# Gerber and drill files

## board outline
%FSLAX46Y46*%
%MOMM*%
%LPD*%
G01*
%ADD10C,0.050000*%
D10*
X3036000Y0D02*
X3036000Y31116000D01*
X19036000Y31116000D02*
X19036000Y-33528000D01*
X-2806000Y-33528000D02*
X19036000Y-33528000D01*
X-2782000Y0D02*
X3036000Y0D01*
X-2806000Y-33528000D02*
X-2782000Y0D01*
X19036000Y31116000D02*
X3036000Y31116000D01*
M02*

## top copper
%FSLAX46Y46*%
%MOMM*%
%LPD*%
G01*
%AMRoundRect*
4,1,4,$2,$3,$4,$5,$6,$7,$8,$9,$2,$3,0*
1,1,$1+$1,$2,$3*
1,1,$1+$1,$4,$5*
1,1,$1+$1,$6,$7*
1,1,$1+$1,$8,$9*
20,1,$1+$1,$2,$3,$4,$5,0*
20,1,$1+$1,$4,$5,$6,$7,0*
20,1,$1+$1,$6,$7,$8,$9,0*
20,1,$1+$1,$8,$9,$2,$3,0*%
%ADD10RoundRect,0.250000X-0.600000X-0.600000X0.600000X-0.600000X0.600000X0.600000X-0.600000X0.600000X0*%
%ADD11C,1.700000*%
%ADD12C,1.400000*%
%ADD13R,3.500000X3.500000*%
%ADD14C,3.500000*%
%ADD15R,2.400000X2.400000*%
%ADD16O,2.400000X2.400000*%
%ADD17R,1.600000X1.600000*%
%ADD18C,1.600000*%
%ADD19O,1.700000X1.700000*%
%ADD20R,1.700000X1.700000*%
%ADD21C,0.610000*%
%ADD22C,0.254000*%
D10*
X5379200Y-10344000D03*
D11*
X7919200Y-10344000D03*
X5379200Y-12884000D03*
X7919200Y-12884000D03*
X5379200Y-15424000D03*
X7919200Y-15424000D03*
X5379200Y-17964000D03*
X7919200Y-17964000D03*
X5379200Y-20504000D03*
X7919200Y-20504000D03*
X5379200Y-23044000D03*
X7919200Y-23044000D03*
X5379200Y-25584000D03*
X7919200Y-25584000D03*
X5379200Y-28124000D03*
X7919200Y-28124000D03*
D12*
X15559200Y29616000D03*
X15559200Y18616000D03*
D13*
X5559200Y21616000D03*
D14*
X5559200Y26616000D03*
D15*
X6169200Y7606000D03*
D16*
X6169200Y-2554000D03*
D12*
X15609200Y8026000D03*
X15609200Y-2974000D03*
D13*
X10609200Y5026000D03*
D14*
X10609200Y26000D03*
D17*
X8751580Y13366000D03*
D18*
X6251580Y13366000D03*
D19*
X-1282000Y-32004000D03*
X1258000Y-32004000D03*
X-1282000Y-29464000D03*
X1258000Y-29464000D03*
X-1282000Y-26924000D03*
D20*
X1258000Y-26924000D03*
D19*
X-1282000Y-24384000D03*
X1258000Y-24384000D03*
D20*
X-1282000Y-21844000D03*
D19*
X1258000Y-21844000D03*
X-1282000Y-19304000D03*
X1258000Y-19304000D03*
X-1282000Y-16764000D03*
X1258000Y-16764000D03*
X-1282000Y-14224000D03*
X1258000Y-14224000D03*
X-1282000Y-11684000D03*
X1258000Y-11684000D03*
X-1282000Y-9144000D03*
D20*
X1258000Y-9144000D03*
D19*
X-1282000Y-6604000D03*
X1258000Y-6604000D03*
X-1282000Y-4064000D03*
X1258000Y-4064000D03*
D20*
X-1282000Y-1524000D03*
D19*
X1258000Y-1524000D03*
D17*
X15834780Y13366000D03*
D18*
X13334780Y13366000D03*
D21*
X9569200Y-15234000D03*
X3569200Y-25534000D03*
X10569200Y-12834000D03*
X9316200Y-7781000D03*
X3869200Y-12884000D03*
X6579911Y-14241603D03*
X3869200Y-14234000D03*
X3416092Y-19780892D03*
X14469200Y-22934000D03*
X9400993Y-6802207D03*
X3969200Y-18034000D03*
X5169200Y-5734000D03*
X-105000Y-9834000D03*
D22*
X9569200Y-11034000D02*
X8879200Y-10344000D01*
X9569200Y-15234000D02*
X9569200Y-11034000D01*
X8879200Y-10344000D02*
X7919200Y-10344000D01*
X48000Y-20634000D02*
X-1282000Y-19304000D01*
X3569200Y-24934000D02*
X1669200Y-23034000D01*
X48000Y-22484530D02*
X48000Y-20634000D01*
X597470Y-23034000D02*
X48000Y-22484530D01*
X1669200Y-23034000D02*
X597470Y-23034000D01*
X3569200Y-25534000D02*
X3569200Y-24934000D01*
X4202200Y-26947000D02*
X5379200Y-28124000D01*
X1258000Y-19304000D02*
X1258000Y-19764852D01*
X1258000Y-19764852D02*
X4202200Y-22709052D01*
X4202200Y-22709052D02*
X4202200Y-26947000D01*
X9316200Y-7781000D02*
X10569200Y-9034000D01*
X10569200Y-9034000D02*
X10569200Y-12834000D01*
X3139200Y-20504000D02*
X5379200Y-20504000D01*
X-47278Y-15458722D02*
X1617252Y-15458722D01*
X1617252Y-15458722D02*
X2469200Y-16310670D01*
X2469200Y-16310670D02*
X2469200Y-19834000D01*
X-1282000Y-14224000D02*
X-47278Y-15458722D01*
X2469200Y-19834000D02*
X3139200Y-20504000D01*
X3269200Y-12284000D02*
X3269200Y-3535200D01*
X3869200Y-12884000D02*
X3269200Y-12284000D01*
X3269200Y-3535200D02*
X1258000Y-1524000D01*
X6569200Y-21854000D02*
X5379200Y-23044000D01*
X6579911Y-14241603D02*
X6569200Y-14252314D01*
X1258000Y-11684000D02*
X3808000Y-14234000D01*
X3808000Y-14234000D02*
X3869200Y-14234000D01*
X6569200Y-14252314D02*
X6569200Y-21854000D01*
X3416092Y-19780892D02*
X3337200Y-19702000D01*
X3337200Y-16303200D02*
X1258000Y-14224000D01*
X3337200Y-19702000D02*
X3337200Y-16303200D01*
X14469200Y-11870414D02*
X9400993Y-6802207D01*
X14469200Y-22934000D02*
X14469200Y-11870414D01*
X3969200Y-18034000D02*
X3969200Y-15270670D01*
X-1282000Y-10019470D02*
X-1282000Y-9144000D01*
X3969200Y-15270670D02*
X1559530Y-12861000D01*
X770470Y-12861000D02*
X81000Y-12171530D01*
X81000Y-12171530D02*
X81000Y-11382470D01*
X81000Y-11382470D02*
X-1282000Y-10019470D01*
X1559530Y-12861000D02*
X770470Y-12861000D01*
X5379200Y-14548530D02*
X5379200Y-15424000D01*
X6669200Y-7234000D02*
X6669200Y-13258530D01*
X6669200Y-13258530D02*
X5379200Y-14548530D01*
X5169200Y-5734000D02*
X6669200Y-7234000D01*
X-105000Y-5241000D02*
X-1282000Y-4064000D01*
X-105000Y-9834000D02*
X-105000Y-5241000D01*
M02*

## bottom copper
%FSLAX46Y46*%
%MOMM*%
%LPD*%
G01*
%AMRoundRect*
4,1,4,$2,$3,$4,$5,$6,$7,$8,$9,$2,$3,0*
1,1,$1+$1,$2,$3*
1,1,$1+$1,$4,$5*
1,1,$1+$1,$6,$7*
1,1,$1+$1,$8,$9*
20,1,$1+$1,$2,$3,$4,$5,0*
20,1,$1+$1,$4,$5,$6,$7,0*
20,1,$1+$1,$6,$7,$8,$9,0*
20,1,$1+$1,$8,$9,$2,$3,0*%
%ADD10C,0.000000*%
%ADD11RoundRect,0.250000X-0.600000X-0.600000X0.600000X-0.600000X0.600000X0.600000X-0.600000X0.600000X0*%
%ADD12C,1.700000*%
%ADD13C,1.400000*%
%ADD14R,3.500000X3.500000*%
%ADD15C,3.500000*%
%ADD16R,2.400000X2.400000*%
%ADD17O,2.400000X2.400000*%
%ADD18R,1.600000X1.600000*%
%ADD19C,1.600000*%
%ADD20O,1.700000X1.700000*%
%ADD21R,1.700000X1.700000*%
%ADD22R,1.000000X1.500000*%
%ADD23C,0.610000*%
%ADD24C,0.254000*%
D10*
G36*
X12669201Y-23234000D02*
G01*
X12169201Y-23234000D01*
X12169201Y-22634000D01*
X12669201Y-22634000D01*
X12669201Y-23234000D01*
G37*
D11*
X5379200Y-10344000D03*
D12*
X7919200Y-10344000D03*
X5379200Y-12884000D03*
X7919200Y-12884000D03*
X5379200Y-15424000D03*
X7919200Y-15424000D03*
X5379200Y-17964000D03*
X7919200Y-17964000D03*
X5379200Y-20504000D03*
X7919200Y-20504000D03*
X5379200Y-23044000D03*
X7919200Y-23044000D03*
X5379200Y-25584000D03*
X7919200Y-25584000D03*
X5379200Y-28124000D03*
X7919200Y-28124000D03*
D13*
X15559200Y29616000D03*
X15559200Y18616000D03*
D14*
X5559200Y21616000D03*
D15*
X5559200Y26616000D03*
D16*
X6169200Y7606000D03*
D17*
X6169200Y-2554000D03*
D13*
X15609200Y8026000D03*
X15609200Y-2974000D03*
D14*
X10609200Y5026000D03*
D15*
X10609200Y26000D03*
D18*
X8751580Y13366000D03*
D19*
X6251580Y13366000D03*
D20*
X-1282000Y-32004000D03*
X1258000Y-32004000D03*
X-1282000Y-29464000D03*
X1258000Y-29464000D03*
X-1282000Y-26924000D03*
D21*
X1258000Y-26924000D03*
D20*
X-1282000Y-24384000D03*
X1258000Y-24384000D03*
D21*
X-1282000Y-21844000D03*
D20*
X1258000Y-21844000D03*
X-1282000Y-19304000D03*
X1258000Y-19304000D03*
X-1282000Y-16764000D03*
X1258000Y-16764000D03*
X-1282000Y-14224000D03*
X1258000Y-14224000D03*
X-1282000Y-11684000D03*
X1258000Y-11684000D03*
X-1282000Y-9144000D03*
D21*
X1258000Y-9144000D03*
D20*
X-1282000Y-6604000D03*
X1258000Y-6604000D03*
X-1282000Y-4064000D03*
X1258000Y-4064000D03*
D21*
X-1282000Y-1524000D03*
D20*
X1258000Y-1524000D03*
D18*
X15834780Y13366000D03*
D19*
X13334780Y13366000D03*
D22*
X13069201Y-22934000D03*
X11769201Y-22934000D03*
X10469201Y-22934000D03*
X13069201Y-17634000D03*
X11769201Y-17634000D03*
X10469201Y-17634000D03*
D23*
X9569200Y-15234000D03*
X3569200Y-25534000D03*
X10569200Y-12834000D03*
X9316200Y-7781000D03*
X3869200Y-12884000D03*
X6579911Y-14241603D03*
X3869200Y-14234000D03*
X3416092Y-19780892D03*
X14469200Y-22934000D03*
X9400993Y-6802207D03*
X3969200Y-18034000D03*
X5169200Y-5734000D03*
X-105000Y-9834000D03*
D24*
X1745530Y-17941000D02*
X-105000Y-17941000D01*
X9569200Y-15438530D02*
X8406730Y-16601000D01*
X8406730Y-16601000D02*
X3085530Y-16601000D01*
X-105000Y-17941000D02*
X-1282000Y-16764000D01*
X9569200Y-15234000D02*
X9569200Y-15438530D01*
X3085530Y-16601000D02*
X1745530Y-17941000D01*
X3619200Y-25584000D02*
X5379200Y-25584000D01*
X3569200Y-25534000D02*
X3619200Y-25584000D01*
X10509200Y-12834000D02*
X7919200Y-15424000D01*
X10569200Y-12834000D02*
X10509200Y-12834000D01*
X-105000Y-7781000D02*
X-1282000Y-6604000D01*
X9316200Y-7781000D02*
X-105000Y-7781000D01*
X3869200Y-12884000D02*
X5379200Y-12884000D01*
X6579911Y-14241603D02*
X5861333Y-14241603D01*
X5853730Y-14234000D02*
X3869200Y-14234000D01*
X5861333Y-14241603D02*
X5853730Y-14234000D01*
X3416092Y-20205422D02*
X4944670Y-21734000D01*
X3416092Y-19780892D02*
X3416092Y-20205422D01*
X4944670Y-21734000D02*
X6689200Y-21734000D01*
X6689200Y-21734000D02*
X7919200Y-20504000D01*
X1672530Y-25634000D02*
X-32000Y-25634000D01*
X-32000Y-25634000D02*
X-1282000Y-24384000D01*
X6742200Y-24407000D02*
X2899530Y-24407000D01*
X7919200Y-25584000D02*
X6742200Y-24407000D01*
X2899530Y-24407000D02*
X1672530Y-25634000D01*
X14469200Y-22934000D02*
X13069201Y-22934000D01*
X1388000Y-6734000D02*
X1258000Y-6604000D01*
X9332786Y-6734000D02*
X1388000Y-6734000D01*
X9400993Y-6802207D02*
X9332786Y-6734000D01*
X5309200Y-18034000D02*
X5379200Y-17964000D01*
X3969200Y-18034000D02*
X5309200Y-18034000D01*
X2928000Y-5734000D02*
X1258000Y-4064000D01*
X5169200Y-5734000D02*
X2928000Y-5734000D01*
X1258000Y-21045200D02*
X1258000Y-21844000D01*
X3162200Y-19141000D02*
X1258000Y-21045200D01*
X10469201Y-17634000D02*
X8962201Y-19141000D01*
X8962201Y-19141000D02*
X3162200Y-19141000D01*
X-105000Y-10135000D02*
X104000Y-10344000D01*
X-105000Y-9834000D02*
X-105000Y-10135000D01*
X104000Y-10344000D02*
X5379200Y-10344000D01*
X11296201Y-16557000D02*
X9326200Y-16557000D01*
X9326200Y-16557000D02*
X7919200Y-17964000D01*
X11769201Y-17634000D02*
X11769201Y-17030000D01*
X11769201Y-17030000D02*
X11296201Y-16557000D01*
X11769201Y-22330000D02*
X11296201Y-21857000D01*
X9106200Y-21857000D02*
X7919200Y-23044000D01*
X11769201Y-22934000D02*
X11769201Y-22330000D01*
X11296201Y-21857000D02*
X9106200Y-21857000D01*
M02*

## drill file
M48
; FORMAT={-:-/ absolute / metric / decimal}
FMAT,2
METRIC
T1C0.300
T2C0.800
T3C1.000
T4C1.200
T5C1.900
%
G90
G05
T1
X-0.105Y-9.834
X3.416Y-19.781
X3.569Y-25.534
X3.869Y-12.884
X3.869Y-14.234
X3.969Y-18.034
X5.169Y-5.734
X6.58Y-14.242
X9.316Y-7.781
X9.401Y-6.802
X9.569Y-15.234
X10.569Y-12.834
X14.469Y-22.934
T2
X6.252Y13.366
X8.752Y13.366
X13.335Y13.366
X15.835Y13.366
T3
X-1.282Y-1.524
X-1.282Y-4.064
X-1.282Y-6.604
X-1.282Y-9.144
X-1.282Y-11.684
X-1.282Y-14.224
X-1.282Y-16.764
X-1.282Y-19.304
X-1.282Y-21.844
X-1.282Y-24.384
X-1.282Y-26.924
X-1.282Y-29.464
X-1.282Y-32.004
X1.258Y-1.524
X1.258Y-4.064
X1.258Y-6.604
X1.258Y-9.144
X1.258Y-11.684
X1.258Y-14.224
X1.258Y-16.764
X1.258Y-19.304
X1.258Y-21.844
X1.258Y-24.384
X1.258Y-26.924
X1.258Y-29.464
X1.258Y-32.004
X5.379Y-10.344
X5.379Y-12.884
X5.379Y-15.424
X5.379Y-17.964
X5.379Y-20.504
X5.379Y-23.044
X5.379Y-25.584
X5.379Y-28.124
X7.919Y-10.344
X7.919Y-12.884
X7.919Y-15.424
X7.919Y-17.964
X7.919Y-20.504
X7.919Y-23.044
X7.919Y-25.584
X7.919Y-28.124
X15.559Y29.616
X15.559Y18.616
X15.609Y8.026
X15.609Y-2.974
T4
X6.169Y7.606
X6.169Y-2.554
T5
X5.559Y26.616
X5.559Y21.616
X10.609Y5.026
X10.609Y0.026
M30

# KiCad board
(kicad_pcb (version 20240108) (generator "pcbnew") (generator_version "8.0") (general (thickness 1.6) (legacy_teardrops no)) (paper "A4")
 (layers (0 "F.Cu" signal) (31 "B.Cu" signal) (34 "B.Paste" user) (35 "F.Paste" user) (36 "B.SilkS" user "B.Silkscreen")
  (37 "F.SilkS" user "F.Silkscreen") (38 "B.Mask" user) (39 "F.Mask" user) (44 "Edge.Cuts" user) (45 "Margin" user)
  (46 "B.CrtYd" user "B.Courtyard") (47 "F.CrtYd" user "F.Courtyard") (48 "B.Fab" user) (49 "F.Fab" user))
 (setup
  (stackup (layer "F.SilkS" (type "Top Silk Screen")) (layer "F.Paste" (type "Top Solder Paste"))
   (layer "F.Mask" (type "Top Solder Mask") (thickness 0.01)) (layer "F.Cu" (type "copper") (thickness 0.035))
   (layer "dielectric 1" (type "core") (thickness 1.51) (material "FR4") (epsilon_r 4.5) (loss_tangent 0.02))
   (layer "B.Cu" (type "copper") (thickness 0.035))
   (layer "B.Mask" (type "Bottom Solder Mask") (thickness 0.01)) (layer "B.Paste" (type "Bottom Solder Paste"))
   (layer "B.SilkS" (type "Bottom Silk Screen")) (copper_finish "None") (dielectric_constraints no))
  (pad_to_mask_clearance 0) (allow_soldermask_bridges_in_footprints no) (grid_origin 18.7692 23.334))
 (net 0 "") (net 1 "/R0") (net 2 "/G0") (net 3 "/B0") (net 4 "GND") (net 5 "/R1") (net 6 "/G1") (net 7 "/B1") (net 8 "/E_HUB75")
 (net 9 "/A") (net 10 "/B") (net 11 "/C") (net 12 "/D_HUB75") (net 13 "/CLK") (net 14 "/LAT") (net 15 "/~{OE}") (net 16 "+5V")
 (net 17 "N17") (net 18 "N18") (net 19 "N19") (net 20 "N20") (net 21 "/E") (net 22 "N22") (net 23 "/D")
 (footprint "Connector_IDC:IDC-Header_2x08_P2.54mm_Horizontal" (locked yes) (layer "F.Cu") (at 5.3792 10.344)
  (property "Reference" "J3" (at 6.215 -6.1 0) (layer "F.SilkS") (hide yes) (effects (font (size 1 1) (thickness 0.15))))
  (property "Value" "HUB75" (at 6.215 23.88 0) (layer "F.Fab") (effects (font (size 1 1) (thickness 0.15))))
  (pad "1" thru_hole roundrect (at 0 0) (size 1.7 1.7) (drill 1) (layers "*.Cu" "*.Mask") (remove_unused_layers no)
   (roundrect_rratio 0.147059) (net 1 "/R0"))
  (pad "2" thru_hole circle (at 2.54 0) (size 1.7 1.7) (drill 1) (layers "*.Cu" "*.Mask") (remove_unused_layers no) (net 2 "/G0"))
  (pad "3" thru_hole circle (at 0 2.54) (size 1.7 1.7) (drill 1) (layers "*.Cu" "*.Mask") (remove_unused_layers no) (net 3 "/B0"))
  (pad "4" thru_hole circle (at 2.54 2.54) (size 1.7 1.7) (drill 1) (layers "*.Cu" "*.Mask") (remove_unused_layers no) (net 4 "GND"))
  (pad "5" thru_hole circle (at 0 5.08) (size 1.7 1.7) (drill 1) (layers "*.Cu" "*.Mask") (remove_unused_layers no) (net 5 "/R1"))
  (pad "6" thru_hole circle (at 2.54 5.08) (size 1.7 1.7) (drill 1) (layers "*.Cu" "*.Mask") (remove_unused_layers no) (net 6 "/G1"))
  (pad "7" thru_hole circle (at 0 7.62) (size 1.7 1.7) (drill 1) (layers "*.Cu" "*.Mask") (remove_unused_layers no) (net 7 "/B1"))
  (pad "8" thru_hole circle (at 2.54 7.62) (size 1.7 1.7) (drill 1) (layers "*.Cu" "*.Mask") (remove_unused_layers no) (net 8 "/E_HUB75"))
  (pad "9" thru_hole circle (at 0 10.16) (size 1.7 1.7) (drill 1) (layers "*.Cu" "*.Mask") (remove_unused_layers no) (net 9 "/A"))
  (pad "10" thru_hole circle (at 2.54 10.16) (size 1.7 1.7) (drill 1) (layers "*.Cu" "*.Mask") (remove_unused_layers no) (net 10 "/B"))
  (pad "11" thru_hole circle (at 0 12.7) (size 1.7 1.7) (drill 1) (layers "*.Cu" "*.Mask") (remove_unused_layers no) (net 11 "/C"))
  (pad "12" thru_hole circle (at 2.54 12.7) (size 1.7 1.7) (drill 1) (layers "*.Cu" "*.Mask") (remove_unused_layers no) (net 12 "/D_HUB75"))
  (pad "13" thru_hole circle (at 0 15.24) (size 1.7 1.7) (drill 1) (layers "*.Cu" "*.Mask") (remove_unused_layers no) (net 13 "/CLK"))
  (pad "14" thru_hole circle (at 2.54 15.24) (size 1.7 1.7) (drill 1) (layers "*.Cu" "*.Mask") (remove_unused_layers no) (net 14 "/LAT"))
  (pad "15" thru_hole circle (at 0 17.78) (size 1.7 1.7) (drill 1) (layers "*.Cu" "*.Mask") (remove_unused_layers no) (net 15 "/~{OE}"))
  (pad "16" thru_hole circle (at 2.54 17.78) (size 1.7 1.7) (drill 1) (layers "*.Cu" "*.Mask") (remove_unused_layers no) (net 4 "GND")))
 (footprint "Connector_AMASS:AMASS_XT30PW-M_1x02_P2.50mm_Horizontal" (layer "F.Cu") (at 5.5592 -21.616 -90)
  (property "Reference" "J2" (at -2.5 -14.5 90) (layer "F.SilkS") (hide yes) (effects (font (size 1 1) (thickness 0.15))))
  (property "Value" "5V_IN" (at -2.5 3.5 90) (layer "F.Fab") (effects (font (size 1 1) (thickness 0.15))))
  (pad "" thru_hole circle (at -8 -10 270) (size 1.4 1.4) (drill 1) (layers "*.Cu" "*.Mask") (remove_unused_layers no))
  (pad "" thru_hole circle (at 3 -10 270) (size 1.4 1.4) (drill 1) (layers "*.Cu" "*.Mask") (remove_unused_layers no))
  (pad "1" thru_hole rect (at 0 0 270) (size 3.5 3.5) (drill 1.9) (layers "*.Cu" "*.Mask") (remove_unused_layers no) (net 4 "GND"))
  (pad "2" thru_hole circle (at -5 0 270) (size 3.5 3.5) (drill 1.9) (layers "*.Cu" "*.Mask") (remove_unused_layers no) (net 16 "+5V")))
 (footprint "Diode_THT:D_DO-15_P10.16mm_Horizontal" (layer "F.Cu") (at 6.1692 -7.606 -90)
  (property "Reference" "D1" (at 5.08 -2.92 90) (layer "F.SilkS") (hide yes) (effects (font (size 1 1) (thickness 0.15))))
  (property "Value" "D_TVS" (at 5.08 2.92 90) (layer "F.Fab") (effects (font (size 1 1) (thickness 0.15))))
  (pad "1" thru_hole rect (at 0 0 270) (size 2.4 2.4) (drill 1.2) (layers "*.Cu" "*.Mask") (remove_unused_layers no) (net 4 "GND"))
  (pad "2" thru_hole oval (at 10.16 0 270) (size 2.4 2.4) (drill 1.2) (layers "*.Cu" "*.Mask") (remove_unused_layers no) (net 16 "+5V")))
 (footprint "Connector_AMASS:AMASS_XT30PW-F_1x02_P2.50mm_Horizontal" (layer "F.Cu") (at 10.6092 -5.026 -90)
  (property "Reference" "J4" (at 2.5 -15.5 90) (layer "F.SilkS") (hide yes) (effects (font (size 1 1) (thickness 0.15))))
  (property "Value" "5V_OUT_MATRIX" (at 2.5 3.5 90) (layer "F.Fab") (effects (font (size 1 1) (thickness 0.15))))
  (pad "" thru_hole circle (at -3 -5) (size 1.4 1.4) (drill 1) (layers "*.Cu" "*.Mask") (remove_unused_layers no))
  (pad "" thru_hole circle (at 8 -5 270) (size 1.4 1.4) (drill 1) (layers "*.Cu" "*.Mask") (remove_unused_layers no))
  (pad "1" thru_hole rect (at 0 0 270) (size 3.5 3.5) (drill 1.9) (layers "*.Cu" "*.Mask") (remove_unused_layers no) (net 4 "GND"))
  (pad "2" thru_hole circle (at 5 0 270) (size 3.5 3.5) (drill 1.9) (layers "*.Cu" "*.Mask") (remove_unused_layers no) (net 16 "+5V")))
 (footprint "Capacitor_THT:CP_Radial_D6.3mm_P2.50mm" (layer "F.Cu") (at 8.75158 -13.366 180)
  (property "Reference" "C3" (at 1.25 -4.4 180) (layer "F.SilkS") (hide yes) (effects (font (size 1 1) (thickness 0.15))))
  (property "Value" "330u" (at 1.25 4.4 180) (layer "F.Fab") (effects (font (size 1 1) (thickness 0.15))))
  (pad "1" thru_hole rect (at 0 0 180) (size 1.6 1.6) (drill 0.8) (layers "*.Cu" "*.Mask") (remove_unused_layers no) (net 16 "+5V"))
  (pad "2" thru_hole circle (at 2.5 0 180) (size 1.6 1.6) (drill 0.8) (layers "*.Cu" "*.Mask") (remove_unused_layers no) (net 4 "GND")))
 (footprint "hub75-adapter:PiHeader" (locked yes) (layer "F.Cu") (at -1.282 1.524)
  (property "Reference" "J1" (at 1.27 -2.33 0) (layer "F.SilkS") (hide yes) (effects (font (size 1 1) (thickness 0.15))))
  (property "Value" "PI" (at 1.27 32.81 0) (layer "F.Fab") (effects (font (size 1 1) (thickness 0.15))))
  (pad "1" thru_hole oval (at 0 30.48 180) (size 1.7 1.7) (drill 1) (layers "*.Cu" "*.Mask") (remove_unused_layers no) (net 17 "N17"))
  (pad "2" thru_hole oval (at 2.54 30.48 180) (size 1.7 1.7) (drill 1) (layers "*.Cu" "*.Mask") (remove_unused_layers no) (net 16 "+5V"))
  (pad "3" thru_hole oval (at 0 27.94 180) (size 1.7 1.7) (drill 1) (layers "*.Cu" "*.Mask") (remove_unused_layers no) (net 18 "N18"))
  (pad "4" thru_hole oval (at 2.54 27.94 180) (size 1.7 1.7) (drill 1) (layers "*.Cu" "*.Mask") (remove_unused_layers no) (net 16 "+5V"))
  (pad "5" thru_hole oval (at 0 25.4 180) (size 1.7 1.7) (drill 1) (layers "*.Cu" "*.Mask") (remove_unused_layers no) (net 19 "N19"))
  (pad "6" thru_hole rect (at 2.54 25.4 180) (size 1.7 1.7) (drill 1) (layers "*.Cu" "*.Mask") (remove_unused_layers no) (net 4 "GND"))
  (pad "7" thru_hole oval (at 0 22.86 180) (size 1.7 1.7) (drill 1) (layers "*.Cu" "*.Mask") (remove_unused_layers no) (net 14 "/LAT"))
  (pad "8" thru_hole oval (at 2.54 22.86 180) (size 1.7 1.7) (drill 1) (layers "*.Cu" "*.Mask") (remove_unused_layers no) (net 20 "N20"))
  (pad "9" thru_hole rect (at 0 20.32 180) (size 1.7 1.7) (drill 1) (layers "*.Cu" "*.Mask") (remove_unused_layers no) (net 4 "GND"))
  (pad "10" thru_hole oval (at 2.54 20.32 180) (size 1.7 1.7) (drill 1) (layers "*.Cu" "*.Mask") (remove_unused_layers no) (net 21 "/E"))
  (pad "11" thru_hole oval (at 0 17.78 180) (size 1.7 1.7) (drill 1) (layers "*.Cu" "*.Mask") (remove_unused_layers no) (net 13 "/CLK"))
  (pad "12" thru_hole oval (at 2.54 17.78 180) (size 1.7 1.7) (drill 1) (layers "*.Cu" "*.Mask") (remove_unused_layers no) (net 15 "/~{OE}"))
  (pad "13" thru_hole oval (at 0 15.24 180) (size 1.7 1.7) (drill 1) (layers "*.Cu" "*.Mask") (remove_unused_layers no) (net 2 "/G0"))
  (pad "14" thru_hole oval (at 2.54 15.24 180) (size 1.7 1.7) (drill 1) (layers "*.Cu" "*.Mask") (remove_unused_layers no) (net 4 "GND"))
  (pad "15" thru_hole oval (at 0 12.7 180) (size 1.7 1.7) (drill 1) (layers "*.Cu" "*.Mask") (remove_unused_layers no) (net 9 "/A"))
  (pad "16" thru_hole oval (at 2.54 12.7 180) (size 1.7 1.7) (drill 1) (layers "*.Cu" "*.Mask") (remove_unused_layers no) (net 10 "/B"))
  (pad "17" thru_hole oval (at 0 10.16 180) (size 1.7 1.7) (drill 1) (layers "*.Cu" "*.Mask") (remove_unused_layers no) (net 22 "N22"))
  (pad "18" thru_hole oval (at 2.54 10.16 180) (size 1.7 1.7) (drill 1) (layers "*.Cu" "*.Mask") (remove_unused_layers no) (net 11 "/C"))
  (pad "19" thru_hole oval (at 0 7.62 180) (size 1.7 1.7) (drill 1) (layers "*.Cu" "*.Mask") (remove_unused_layers no) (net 7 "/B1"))
  (pad "20" thru_hole rect (at 2.54 7.62 180) (size 1.7 1.7) (drill 1) (layers "*.Cu" "*.Mask") (remove_unused_layers no) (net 4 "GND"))
  (pad "21" thru_hole oval (at 0 5.08 180) (size 1.7 1.7) (drill 1) (layers "*.Cu" "*.Mask") (remove_unused_layers no) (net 6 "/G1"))
  (pad "22" thru_hole oval (at 2.54 5.08 180) (size 1.7 1.7) (drill 1) (layers "*.Cu" "*.Mask") (remove_unused_layers no) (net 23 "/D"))
  (pad "23" thru_hole oval (at 0 2.54 180) (size 1.7 1.7) (drill 1) (layers "*.Cu" "*.Mask") (remove_unused_layers no) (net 1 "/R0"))
  (pad "24" thru_hole oval (at 2.54 2.54 180) (size 1.7 1.7) (drill 1) (layers "*.Cu" "*.Mask") (remove_unused_layers no) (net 5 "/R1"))
  (pad "25" thru_hole rect (at 0 0 180) (size 1.7 1.7) (drill 1) (layers "*.Cu" "*.Mask") (remove_unused_layers no) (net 4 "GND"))
  (pad "26" thru_hole oval (at 2.54 0 180) (size 1.7 1.7) (drill 1) (layers "*.Cu" "*.Mask") (remove_unused_layers no) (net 3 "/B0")))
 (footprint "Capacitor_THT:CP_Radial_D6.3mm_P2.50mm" (layer "F.Cu") (at 15.83478 -13.366 180)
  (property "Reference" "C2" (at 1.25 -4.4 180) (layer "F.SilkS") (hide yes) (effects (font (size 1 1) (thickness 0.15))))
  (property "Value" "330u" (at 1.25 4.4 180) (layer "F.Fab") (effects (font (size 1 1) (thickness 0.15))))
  (pad "1" thru_hole rect (at 0 0 180) (size 1.6 1.6) (drill 0.8) (layers "*.Cu" "*.Mask") (remove_unused_layers no) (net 16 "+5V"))
  (pad "2" thru_hole circle (at 2.5 0 180) (size 1.6 1.6) (drill 0.8) (layers "*.Cu" "*.Mask") (remove_unused_layers no) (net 4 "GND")))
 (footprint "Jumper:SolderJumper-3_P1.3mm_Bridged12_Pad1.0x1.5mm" (layer "B.Cu") (at 11.769201 22.934 180)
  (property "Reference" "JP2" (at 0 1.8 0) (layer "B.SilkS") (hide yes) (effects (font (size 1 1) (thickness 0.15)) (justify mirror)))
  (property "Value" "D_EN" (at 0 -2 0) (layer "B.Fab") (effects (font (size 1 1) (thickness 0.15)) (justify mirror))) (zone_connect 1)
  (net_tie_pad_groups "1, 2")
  (fp_poly (pts (xy -0.9 0.3) (xy -0.4 0.3) (xy -0.4 -0.3) (xy -0.9 -0.3)) (stroke (width 0) (type solid)) (fill solid) (layer "B.Cu"))
  (pad "1" smd rect (at -1.3 0 180) (size 1 1.5) (layers "B.Cu" "B.Mask") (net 23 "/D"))
  (pad "2" smd rect (at 0 0 180) (size 1 1.5) (layers "B.Cu" "B.Mask") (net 12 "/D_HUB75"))
  (pad "3" smd rect (at 1.3 0 180) (size 1 1.5) (layers "B.Cu" "B.Mask") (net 4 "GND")))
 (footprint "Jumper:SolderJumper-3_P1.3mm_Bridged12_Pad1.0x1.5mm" (layer "B.Cu") (at 11.769201 17.634 180)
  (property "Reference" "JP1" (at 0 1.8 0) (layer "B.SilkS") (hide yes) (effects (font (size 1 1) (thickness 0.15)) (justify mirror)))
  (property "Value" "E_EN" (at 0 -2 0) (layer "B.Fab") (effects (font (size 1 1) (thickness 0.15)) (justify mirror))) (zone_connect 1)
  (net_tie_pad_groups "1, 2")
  (pad "1" smd rect (at -1.3 0 180) (size 1 1.5) (layers "B.Cu" "B.Mask") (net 4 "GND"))
  (pad "2" smd rect (at 0 0 180) (size 1 1.5) (layers "B.Cu" "B.Mask") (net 8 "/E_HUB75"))
  (pad "3" smd rect (at 1.3 0 180) (size 1 1.5) (layers "B.Cu" "B.Mask") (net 21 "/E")))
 (gr_line (start 3.036 0) (end 3.036 -31.116) (stroke (width 0.05) (type default)) (layer "Edge.Cuts"))
 (gr_line (start 19.036 -31.116) (end 19.036 33.528) (stroke (width 0.05) (type default)) (layer "Edge.Cuts"))
 (gr_line (start -2.806 33.528) (end 19.036 33.528) (stroke (width 0.05) (type default)) (layer "Edge.Cuts"))
 (gr_line (start -2.782 0) (end 3.036 0) (stroke (width 0.05) (type default)) (layer "Edge.Cuts"))
 (gr_line (start -2.806 33.528) (end -2.782 0) (locked yes) (stroke (width 0.05) (type default)) (layer "Edge.Cuts"))
 (gr_line (start 19.036 -31.116) (end 3.036 -31.116) (stroke (width 0.05) (type default)) (layer "Edge.Cuts"))
 (segment (start 9.5692 11.034) (end 8.8792 10.344) (width 0.254) (layer "F.Cu") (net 2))
 (segment (start 9.5692 15.234) (end 9.5692 11.034) (width 0.254) (layer "F.Cu") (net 2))
 (segment (start 8.8792 10.344) (end 7.9192 10.344) (width 0.254) (layer "F.Cu") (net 2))
 (via (at 9.5692 15.234) (size 0.61) (drill 0.3) (layers "F.Cu" "B.Cu") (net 2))
 (segment (start 1.74553 17.941) (end -0.105 17.941) (width 0.254) (layer "B.Cu") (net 2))
 (segment (start 9.5692 15.43853) (end 8.40673 16.601) (width 0.254) (layer "B.Cu") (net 2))
 (segment (start 8.40673 16.601) (end 3.08553 16.601) (width 0.254) (layer "B.Cu") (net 2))
 (segment (start -0.105 17.941) (end -1.282 16.764) (width 0.254) (layer "B.Cu") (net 2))
 (segment (start 9.5692 15.234) (end 9.5692 15.43853) (width 0.254) (layer "B.Cu") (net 2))
 (segment (start 3.08553 16.601) (end 1.74553 17.941) (width 0.254) (layer "B.Cu") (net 2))
 (segment (start 0.048 20.634) (end -1.282 19.304) (width 0.254) (layer "F.Cu") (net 13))
 (segment (start 3.5692 24.934) (end 1.6692 23.034) (width 0.254) (layer "F.Cu") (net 13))
 (segment (start 0.048 22.48453) (end 0.048 20.634) (width 0.254) (layer "F.Cu") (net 13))
 (segment (start 0.59747 23.034) (end 0.048 22.48453) (width 0.254) (layer "F.Cu") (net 13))
 (segment (start 1.6692 23.034) (end 0.59747 23.034) (width 0.254) (layer "F.Cu") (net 13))
 (segment (start 3.5692 25.534) (end 3.5692 24.934) (width 0.254) (layer "F.Cu") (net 13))
 (via (at 3.5692 25.534) (size 0.61) (drill 0.3) (layers "F.Cu" "B.Cu") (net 13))
 (segment (start 3.6192 25.584) (end 5.3792 25.584) (width 0.254) (layer "B.Cu") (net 13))
 (segment (start 3.5692 25.534) (end 3.6192 25.584) (width 0.254) (layer "B.Cu") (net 13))
 (segment (start 4.2022 26.947) (end 5.3792 28.124) (width 0.254) (layer "F.Cu") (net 15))
 (segment (start 1.258 19.304) (end 1.258 19.764852) (width 0.254) (layer "F.Cu") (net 15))
 (segment (start 1.258 19.764852) (end 4.2022 22.709052) (width 0.254) (layer "F.Cu") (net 15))
 (segment (start 4.2022 22.709052) (end 4.2022 26.947) (width 0.254) (layer "F.Cu") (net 15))
 (segment (start 9.3162 7.781) (end 10.5692 9.034) (width 0.254) (layer "F.Cu") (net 6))
 (segment (start 10.5692 9.034) (end 10.5692 12.834) (width 0.254) (layer "F.Cu") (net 6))
 (via (at 10.5692 12.834) (size 0.61) (drill 0.3) (layers "F.Cu" "B.Cu") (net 6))
 (via (at 9.3162 7.781) (size 0.61) (drill 0.3) (layers "F.Cu" "B.Cu") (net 6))
 (segment (start 10.5092 12.834) (end 7.9192 15.424) (width 0.254) (layer "B.Cu") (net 6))
 (segment (start 10.5692 12.834) (end 10.5092 12.834) (width 0.254) (layer "B.Cu") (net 6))
 (segment (start -0.105 7.781) (end -1.282 6.604) (width 0.254) (layer "B.Cu") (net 6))
 (segment (start 9.3162 7.781) (end -0.105 7.781) (width 0.254) (layer "B.Cu") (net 6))
 (segment (start 3.1392 20.504) (end 5.3792 20.504) (width 0.254) (layer "F.Cu") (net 9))
 (segment (start -0.047278 15.458722) (end 1.617252 15.458722) (width 0.254) (layer "F.Cu") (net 9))
 (segment (start 1.617252 15.458722) (end 2.4692 16.31067) (width 0.254) (layer "F.Cu") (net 9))
 (segment (start 2.4692 16.31067) (end 2.4692 19.834) (width 0.254) (layer "F.Cu") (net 9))
 (segment (start -1.282 14.224) (end -0.047278 15.458722) (width 0.254) (layer "F.Cu") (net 9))
 (segment (start 2.4692 19.834) (end 3.1392 20.504) (width 0.254) (layer "F.Cu") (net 9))
 (segment (start 3.2692 12.284) (end 3.2692 3.5352) (width 0.254) (layer "F.Cu") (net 3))
 (segment (start 3.8692 12.884) (end 3.2692 12.284) (width 0.254) (layer "F.Cu") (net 3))
 (segment (start 3.2692 3.5352) (end 1.258 1.524) (width 0.254) (layer "F.Cu") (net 3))
 (via (at 3.8692 12.884) (size 0.61) (drill 0.3) (layers "F.Cu" "B.Cu") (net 3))
 (segment (start 3.8692 12.884) (end 5.3792 12.884) (width 0.254) (layer "B.Cu") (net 3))
 (segment (start 6.5692 21.854) (end 5.3792 23.044) (width 0.254) (layer "F.Cu") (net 11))
 (segment (start 6.579911 14.241603) (end 6.5692 14.252314) (width 0.254) (layer "F.Cu") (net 11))
 (segment (start 1.258 11.684) (end 3.808 14.234) (width 0.254) (layer "F.Cu") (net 11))
 (segment (start 3.808 14.234) (end 3.8692 14.234) (width 0.254) (layer "F.Cu") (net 11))
 (segment (start 6.5692 14.252314) (end 6.5692 21.854) (width 0.254) (layer "F.Cu") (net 11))
 (via (at 6.579911 14.241603) (size 0.61) (drill 0.3) (layers "F.Cu" "B.Cu") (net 11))
 (via (at 3.8692 14.234) (size 0.61) (drill 0.3) (layers "F.Cu" "B.Cu") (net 11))
 (segment (start 6.579911 14.241603) (end 5.861333 14.241603) (width 0.254) (layer "B.Cu") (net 11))
 (segment (start 5.85373 14.234) (end 3.8692 14.234) (width 0.254) (layer "B.Cu") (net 11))
 (segment (start 5.861333 14.241603) (end 5.85373 14.234) (width 0.254) (layer "B.Cu") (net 11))
 (segment (start 3.416092 19.780892) (end 3.3372 19.702) (width 0.254) (layer "F.Cu") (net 10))
 (segment (start 3.3372 16.3032) (end 1.258 14.224) (width 0.254) (layer "F.Cu") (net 10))
 (segment (start 3.3372 19.702) (end 3.3372 16.3032) (width 0.254) (layer "F.Cu") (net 10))
 (via (at 3.416092 19.780892) (size 0.61) (drill 0.3) (layers "F.Cu" "B.Cu") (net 10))
 (segment (start 3.416092 20.205422) (end 4.94467 21.734) (width 0.254) (layer "B.Cu") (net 10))
 (segment (start 3.416092 19.780892) (end 3.416092 20.205422) (width 0.254) (layer "B.Cu") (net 10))
 (segment (start 4.94467 21.734) (end 6.6892 21.734) (width 0.254) (layer "B.Cu") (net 10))
 (segment (start 6.6892 21.734) (end 7.9192 20.504) (width 0.254) (layer "B.Cu") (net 10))
 (segment (start 1.67253 25.634) (end -0.032 25.634) (width 0.254) (layer "B.Cu") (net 14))
 (segment (start -0.032 25.634) (end -1.282 24.384) (width 0.254) (layer "B.Cu") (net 14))
 (segment (start 6.7422 24.407) (end 2.89953 24.407) (width 0.254) (layer "B.Cu") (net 14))
 (segment (start 7.9192 25.584) (end 6.7422 24.407) (width 0.254) (layer "B.Cu") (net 14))
 (segment (start 2.89953 24.407) (end 1.67253 25.634) (width 0.254) (layer "B.Cu") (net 14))
 (segment (start 14.4692 11.870414) (end 9.400993 6.802207) (width 0.254) (layer "F.Cu") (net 23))
 (segment (start 14.4692 22.934) (end 14.4692 11.870414) (width 0.254) (layer "F.Cu") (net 23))
 (via (at 14.4692 22.934) (size 0.61) (drill 0.3) (layers "F.Cu" "B.Cu") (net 23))
 (via (at 9.400993 6.802207) (size 0.61) (drill 0.3) (layers "F.Cu" "B.Cu") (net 23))
 (segment (start 14.4692 22.934) (end 13.069201 22.934) (width 0.254) (layer "B.Cu") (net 23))
 (segment (start 1.388 6.734) (end 1.258 6.604) (width 0.254) (layer "B.Cu") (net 23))
 (segment (start 9.332786 6.734) (end 1.388 6.734) (width 0.254) (layer "B.Cu") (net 23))
 (segment (start 9.400993 6.802207) (end 9.332786 6.734) (width 0.254) (layer "B.Cu") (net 23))
 (segment (start 3.9692 18.034) (end 3.9692 15.27067) (width 0.254) (layer "F.Cu") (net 7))
 (segment (start -1.282 10.01947) (end -1.282 9.144) (width 0.254) (layer "F.Cu") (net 7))
 (segment (start 3.9692 15.27067) (end 1.55953 12.861) (width 0.254) (layer "F.Cu") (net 7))
 (segment (start 0.77047 12.861) (end 0.081 12.17153) (width 0.254) (layer "F.Cu") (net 7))
 (segment (start 0.081 12.17153) (end 0.081 11.38247) (width 0.254) (layer "F.Cu") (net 7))
 (segment (start 0.081 11.38247) (end -1.282 10.01947) (width 0.254) (layer "F.Cu") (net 7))
 (segment (start 1.55953 12.861) (end 0.77047 12.861) (width 0.254) (layer "F.Cu") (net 7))
 (via (at 3.9692 18.034) (size 0.61) (drill 0.3) (layers "F.Cu" "B.Cu") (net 7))
 (segment (start 5.3092 18.034) (end 5.3792 17.964) (width 0.254) (layer "B.Cu") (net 7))
 (segment (start 3.9692 18.034) (end 5.3092 18.034) (width 0.254) (layer "B.Cu") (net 7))
 (segment (start 5.3792 14.54853) (end 5.3792 15.424) (width 0.254) (layer "F.Cu") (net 5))
 (segment (start 6.6692 7.234) (end 6.6692 13.25853) (width 0.254) (layer "F.Cu") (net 5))
 (segment (start 6.6692 13.25853) (end 5.3792 14.54853) (width 0.254) (layer "F.Cu") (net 5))
 (segment (start 5.1692 5.734) (end 6.6692 7.234) (width 0.254) (layer "F.Cu") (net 5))
 (via (at 5.1692 5.734) (size 0.61) (drill 0.3) (layers "F.Cu" "B.Cu") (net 5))
 (segment (start 2.928 5.734) (end 1.258 4.064) (width 0.254) (layer "B.Cu") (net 5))
 (segment (start 5.1692 5.734) (end 2.928 5.734) (width 0.254) (layer "B.Cu") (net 5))
 (segment (start 1.258 21.0452) (end 1.258 21.844) (width 0.254) (layer "B.Cu") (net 21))
 (segment (start 3.1622 19.141) (end 1.258 21.0452) (width 0.254) (layer "B.Cu") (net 21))
 (segment (start 10.469201 17.634) (end 8.962201 19.141) (width 0.254) (layer "B.Cu") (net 21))
 (segment (start 8.962201 19.141) (end 3.1622 19.141) (width 0.254) (layer "B.Cu") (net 21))
 (segment (start -0.105 5.241) (end -1.282 4.064) (width 0.254) (layer "F.Cu") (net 1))
 (segment (start -0.105 9.834) (end -0.105 5.241) (width 0.254) (layer "F.Cu") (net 1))
 (via (at -0.105 9.834) (size 0.61) (drill 0.3) (layers "F.Cu" "B.Cu") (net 1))
 (segment (start -0.105 10.135) (end 0.104 10.344) (width 0.254) (layer "B.Cu") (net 1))
 (segment (start -0.105 9.834) (end -0.105 10.135) (width 0.254) (layer "B.Cu") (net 1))
 (segment (start 0.104 10.344) (end 5.3792 10.344) (width 0.254) (layer "B.Cu") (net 1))
 (segment (start 11.296201 16.557) (end 9.3262 16.557) (width 0.254) (layer "B.Cu") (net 8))
 (segment (start 9.3262 16.557) (end 7.9192 17.964) (width 0.254) (layer "B.Cu") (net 8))
 (segment (start 11.769201 17.634) (end 11.769201 17.03) (width 0.254) (layer "B.Cu") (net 8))
 (segment (start 11.769201 17.03) (end 11.296201 16.557) (width 0.254) (layer "B.Cu") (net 8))
 (segment (start 11.769201 22.33) (end 11.296201 21.857) (width 0.254) (layer "B.Cu") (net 12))
 (segment (start 9.1062 21.857) (end 7.9192 23.044) (width 0.254) (layer "B.Cu") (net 12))
 (segment (start 11.769201 22.934) (end 11.769201 22.33) (width 0.254) (layer "B.Cu") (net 12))
 (segment (start 11.296201 21.857) (end 9.1062 21.857) (width 0.254) (layer "B.Cu") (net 12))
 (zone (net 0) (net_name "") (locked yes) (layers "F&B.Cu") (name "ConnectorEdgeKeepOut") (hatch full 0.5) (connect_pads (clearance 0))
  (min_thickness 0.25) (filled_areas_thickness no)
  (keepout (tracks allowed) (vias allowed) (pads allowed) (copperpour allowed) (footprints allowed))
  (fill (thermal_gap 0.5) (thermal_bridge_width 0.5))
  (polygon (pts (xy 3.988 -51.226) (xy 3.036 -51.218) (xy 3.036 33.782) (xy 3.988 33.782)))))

